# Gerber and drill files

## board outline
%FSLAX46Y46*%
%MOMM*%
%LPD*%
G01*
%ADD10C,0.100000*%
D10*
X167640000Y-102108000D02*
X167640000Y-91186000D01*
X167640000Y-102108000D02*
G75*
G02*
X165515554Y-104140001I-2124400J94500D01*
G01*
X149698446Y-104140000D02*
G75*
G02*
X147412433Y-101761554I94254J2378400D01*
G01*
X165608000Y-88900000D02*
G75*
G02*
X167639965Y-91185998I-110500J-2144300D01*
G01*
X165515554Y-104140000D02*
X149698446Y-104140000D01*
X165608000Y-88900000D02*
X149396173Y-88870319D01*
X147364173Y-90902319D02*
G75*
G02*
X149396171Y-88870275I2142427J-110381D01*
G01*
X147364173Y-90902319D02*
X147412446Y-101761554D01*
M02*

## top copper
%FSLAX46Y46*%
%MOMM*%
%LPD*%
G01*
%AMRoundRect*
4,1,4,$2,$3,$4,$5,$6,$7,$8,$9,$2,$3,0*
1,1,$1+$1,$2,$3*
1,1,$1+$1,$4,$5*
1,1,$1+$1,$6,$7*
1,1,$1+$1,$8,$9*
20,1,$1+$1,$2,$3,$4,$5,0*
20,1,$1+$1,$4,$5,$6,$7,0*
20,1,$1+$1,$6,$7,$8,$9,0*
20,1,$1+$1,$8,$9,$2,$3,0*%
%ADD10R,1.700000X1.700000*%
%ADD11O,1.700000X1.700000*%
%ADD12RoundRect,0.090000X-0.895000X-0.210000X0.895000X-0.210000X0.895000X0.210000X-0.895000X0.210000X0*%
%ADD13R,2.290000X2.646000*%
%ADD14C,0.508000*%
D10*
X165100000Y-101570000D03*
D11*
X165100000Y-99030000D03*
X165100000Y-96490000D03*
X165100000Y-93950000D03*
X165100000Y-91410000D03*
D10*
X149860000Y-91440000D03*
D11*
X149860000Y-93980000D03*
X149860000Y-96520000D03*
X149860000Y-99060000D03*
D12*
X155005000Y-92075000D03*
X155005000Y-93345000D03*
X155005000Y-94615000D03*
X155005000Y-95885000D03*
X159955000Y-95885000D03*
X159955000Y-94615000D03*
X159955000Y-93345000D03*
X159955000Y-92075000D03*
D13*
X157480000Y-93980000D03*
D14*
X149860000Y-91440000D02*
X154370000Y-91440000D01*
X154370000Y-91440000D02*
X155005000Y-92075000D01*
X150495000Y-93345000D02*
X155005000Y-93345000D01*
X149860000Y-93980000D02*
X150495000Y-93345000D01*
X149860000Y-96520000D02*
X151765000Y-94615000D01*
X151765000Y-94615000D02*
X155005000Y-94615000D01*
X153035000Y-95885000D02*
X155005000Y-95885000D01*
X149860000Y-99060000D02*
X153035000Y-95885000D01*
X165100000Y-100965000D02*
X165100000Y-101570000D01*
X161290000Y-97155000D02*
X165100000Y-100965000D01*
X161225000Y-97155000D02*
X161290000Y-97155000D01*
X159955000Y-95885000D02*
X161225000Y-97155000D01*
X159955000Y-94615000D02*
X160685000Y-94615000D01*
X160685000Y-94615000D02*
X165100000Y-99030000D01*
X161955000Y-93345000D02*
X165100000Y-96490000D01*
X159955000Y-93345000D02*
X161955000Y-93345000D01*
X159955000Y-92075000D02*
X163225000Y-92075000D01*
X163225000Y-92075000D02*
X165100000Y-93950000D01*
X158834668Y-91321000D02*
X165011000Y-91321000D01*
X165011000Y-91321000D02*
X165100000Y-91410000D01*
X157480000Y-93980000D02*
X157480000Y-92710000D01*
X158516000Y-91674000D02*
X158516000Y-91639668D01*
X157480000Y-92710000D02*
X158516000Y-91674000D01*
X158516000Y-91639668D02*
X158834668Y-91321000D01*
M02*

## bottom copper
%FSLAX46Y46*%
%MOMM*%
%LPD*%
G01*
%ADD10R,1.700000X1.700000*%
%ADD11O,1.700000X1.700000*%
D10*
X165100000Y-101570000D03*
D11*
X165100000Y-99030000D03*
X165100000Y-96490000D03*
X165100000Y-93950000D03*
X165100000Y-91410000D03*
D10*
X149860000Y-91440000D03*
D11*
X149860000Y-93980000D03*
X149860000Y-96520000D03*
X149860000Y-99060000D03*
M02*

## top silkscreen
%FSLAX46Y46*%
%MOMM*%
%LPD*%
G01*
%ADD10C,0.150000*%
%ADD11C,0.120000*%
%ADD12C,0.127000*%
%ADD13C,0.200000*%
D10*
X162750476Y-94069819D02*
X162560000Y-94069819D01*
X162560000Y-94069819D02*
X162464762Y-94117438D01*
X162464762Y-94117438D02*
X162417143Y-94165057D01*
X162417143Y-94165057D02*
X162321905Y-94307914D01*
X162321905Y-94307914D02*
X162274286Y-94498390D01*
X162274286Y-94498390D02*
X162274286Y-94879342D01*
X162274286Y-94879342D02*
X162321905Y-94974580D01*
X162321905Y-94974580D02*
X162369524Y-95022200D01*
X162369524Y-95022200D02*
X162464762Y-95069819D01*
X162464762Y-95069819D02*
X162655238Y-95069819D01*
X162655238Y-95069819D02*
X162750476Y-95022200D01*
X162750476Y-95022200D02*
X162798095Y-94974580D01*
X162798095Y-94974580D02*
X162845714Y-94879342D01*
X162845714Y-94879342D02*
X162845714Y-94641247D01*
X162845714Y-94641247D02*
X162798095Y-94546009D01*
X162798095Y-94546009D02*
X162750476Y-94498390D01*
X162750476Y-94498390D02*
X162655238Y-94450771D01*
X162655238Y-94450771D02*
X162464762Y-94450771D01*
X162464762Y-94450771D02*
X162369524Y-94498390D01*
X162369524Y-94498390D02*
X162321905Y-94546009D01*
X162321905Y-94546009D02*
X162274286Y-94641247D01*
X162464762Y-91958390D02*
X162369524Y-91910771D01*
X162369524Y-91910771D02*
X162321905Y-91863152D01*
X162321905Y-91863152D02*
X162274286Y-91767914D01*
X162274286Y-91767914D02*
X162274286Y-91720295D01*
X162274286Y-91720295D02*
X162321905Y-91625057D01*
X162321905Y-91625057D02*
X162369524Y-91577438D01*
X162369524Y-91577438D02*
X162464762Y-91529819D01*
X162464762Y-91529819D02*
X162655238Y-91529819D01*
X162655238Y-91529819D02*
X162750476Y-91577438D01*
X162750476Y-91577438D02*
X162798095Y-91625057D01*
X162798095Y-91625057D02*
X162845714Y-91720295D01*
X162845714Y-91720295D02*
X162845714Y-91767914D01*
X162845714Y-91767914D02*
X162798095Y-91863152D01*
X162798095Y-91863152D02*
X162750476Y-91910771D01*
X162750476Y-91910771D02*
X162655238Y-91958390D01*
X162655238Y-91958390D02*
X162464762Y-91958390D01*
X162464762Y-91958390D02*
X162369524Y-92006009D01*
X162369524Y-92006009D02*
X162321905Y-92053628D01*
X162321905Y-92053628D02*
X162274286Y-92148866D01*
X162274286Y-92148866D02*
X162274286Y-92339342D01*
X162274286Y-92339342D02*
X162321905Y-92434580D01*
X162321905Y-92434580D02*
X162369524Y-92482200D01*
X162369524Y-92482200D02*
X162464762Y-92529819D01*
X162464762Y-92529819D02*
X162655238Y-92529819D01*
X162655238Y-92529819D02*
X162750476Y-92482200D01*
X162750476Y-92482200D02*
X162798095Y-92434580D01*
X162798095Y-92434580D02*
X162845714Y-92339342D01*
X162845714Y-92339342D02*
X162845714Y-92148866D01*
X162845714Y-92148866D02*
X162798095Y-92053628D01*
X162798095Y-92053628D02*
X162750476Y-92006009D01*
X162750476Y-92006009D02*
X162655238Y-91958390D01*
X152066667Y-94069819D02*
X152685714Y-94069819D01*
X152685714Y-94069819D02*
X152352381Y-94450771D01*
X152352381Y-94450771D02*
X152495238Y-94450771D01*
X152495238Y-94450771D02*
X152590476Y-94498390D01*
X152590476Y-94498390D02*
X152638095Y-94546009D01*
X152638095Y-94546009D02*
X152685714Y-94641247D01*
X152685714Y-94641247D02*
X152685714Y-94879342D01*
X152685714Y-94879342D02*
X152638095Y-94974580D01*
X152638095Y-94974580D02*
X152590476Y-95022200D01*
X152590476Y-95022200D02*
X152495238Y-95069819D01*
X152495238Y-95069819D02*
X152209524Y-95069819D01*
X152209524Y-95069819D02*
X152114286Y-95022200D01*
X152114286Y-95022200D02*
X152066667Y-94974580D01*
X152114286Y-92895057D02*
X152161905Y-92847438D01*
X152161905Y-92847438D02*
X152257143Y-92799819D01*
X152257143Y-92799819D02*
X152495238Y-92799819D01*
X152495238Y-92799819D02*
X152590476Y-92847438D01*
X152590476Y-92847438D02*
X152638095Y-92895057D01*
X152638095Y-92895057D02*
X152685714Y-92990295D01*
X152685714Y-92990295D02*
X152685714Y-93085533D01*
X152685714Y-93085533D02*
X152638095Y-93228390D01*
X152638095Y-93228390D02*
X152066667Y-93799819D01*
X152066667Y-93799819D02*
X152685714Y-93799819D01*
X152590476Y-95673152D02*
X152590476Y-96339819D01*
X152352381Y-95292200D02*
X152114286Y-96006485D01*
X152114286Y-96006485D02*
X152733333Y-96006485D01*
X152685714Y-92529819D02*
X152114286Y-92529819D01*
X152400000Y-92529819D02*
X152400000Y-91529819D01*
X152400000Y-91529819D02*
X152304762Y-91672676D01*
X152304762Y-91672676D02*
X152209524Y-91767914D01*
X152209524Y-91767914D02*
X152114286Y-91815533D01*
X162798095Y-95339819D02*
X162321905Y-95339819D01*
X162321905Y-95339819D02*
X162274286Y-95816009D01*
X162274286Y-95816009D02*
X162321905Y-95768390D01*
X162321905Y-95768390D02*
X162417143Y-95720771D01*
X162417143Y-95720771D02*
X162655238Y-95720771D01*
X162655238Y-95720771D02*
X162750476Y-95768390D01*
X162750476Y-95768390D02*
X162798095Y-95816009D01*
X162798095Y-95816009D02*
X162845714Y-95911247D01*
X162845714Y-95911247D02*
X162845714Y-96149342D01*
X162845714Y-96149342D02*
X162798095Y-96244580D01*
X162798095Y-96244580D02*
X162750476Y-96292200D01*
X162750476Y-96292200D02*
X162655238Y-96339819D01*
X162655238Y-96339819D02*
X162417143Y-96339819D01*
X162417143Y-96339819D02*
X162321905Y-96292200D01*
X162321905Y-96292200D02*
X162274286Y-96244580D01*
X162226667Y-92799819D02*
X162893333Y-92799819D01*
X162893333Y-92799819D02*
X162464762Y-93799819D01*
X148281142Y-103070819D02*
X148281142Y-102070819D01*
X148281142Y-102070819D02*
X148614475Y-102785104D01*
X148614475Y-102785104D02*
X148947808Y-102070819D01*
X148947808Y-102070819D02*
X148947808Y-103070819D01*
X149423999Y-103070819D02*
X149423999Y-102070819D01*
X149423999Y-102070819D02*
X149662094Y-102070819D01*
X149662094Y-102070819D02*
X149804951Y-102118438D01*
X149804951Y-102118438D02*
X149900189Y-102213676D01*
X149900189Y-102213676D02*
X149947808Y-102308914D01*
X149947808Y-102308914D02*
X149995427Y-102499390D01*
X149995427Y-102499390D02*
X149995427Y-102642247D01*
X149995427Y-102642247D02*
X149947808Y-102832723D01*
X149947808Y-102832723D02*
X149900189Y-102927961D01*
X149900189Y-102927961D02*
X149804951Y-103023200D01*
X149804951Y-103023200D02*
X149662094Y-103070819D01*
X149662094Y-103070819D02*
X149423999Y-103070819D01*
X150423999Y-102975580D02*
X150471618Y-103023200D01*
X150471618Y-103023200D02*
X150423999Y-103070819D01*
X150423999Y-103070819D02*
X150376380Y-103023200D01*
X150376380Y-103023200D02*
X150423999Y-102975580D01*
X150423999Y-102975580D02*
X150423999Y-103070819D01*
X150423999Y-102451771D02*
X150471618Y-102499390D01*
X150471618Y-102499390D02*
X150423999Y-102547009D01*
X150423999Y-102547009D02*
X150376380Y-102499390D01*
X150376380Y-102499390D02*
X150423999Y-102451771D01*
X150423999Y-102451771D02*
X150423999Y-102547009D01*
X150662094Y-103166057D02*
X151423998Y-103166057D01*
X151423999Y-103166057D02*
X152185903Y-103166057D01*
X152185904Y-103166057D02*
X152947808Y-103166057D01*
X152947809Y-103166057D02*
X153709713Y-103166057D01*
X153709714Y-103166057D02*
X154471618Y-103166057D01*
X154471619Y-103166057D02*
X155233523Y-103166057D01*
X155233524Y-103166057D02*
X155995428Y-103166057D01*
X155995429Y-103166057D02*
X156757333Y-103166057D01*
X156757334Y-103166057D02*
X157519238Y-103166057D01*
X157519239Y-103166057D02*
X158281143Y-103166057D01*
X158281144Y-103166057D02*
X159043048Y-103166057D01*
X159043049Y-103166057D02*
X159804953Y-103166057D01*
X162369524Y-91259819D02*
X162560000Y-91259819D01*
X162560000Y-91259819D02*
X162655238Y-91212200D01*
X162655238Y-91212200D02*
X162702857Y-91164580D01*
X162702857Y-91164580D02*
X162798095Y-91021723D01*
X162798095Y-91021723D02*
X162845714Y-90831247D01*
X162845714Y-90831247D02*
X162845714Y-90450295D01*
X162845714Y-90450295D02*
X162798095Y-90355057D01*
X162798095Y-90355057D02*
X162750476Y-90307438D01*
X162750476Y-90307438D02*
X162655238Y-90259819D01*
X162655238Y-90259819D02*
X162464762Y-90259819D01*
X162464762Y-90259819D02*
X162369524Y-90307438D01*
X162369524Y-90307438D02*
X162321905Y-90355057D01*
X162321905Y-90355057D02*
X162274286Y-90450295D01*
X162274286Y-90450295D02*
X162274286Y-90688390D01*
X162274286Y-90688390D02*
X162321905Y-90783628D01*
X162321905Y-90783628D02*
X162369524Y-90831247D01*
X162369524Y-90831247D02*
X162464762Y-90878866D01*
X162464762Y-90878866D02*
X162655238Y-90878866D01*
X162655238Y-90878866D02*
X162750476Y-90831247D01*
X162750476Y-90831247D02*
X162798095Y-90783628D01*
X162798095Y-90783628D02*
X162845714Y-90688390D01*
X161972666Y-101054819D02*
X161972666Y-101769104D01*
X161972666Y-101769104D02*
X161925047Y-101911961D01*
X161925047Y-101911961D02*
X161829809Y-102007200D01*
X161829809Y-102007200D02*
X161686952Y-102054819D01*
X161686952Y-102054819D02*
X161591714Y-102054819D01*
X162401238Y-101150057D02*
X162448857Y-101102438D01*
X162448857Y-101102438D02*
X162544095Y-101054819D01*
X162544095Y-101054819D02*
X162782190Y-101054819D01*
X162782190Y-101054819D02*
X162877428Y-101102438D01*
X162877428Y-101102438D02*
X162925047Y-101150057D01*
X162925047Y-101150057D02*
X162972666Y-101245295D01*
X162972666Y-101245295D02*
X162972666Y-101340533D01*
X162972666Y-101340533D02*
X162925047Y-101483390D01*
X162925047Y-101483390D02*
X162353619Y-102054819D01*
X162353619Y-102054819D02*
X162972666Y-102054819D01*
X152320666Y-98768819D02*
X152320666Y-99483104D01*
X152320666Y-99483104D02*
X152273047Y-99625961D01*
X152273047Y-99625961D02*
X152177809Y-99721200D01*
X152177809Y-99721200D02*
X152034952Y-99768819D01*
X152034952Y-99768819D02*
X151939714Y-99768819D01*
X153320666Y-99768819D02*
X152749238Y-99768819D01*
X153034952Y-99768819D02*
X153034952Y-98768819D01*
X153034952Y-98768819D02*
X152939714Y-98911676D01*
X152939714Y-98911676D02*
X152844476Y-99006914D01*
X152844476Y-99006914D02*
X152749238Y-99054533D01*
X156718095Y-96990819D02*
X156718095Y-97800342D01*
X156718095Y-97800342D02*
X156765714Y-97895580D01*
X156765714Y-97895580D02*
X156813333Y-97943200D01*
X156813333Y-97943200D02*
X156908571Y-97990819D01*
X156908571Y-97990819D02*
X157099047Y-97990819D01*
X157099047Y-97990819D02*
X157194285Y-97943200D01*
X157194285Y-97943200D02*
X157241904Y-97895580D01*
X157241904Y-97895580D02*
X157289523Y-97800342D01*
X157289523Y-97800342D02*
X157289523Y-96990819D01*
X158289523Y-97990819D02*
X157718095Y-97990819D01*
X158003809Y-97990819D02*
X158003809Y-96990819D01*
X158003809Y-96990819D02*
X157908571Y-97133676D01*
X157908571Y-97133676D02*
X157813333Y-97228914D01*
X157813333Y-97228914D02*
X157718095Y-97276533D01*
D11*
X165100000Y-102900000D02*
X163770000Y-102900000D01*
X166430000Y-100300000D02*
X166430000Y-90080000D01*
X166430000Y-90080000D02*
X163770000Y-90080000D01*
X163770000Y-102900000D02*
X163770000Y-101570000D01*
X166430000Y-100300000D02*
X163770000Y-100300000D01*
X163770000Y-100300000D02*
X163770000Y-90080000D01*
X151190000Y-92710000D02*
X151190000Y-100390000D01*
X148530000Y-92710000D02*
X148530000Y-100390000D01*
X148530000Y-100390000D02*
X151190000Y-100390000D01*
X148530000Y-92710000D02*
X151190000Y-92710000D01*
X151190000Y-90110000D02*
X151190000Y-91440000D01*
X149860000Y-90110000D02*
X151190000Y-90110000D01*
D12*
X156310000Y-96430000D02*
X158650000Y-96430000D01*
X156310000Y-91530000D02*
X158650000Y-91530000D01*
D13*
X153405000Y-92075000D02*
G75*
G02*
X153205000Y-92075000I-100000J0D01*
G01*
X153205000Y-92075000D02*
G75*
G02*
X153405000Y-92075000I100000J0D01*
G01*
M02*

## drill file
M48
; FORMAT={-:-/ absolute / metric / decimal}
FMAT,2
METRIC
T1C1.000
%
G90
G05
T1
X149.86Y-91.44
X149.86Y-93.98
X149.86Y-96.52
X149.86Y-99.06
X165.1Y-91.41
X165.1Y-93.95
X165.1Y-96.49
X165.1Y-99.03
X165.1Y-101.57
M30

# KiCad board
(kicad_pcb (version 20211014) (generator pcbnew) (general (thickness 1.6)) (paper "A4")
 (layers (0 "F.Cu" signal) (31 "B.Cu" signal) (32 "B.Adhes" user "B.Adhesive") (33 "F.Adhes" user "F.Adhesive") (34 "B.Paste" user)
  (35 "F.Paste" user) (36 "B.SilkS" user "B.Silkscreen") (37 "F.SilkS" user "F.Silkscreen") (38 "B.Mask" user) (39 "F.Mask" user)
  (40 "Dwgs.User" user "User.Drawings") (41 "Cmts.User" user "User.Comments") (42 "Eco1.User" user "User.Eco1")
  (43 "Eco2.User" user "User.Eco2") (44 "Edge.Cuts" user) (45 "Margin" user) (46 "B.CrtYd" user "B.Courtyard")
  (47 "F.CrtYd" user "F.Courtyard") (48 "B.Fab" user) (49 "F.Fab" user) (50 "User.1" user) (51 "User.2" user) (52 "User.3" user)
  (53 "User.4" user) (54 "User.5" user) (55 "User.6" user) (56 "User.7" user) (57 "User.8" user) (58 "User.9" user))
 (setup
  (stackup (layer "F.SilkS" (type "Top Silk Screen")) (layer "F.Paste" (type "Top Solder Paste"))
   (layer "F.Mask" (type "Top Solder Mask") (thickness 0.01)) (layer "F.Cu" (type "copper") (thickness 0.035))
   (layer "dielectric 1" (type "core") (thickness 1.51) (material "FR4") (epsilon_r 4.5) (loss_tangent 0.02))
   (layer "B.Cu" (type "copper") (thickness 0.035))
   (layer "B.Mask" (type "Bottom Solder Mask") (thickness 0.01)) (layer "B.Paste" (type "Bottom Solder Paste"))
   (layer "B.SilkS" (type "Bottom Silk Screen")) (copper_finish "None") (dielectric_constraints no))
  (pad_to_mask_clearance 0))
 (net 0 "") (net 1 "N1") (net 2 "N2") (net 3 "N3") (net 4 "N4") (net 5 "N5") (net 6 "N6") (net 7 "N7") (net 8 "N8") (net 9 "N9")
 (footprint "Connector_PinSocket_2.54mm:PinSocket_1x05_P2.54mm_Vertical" (layer "F.Cu") (at 165.1 101.57 180)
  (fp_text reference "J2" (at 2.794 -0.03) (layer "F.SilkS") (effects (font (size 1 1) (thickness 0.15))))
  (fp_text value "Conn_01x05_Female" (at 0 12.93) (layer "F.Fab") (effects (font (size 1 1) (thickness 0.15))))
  (fp_line (start 0 -1.33) (end 1.33 -1.33) (layer "F.SilkS") (width 0.12))
  (fp_line (start -1.33 1.27) (end -1.33 11.49) (layer "F.SilkS") (width 0.12))
  (fp_line (start -1.33 11.49) (end 1.33 11.49) (layer "F.SilkS") (width 0.12))
  (fp_line (start 1.33 -1.33) (end 1.33 0) (layer "F.SilkS") (width 0.12))
  (fp_line (start -1.33 1.27) (end 1.33 1.27) (layer "F.SilkS") (width 0.12))
  (fp_line (start 1.33 1.27) (end 1.33 11.49) (layer "F.SilkS") (width 0.12))
  (pad "1" thru_hole rect (at 0 0 180) (size 1.7 1.7) (drill 1) (layers *.Cu *.Mask) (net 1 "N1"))
  (pad "2" thru_hole oval (at 0 2.54 180) (size 1.7 1.7) (drill 1) (layers *.Cu *.Mask) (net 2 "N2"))
  (pad "3" thru_hole oval (at 0 5.08 180) (size 1.7 1.7) (drill 1) (layers *.Cu *.Mask) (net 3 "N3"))
  (pad "4" thru_hole oval (at 0 7.62 180) (size 1.7 1.7) (drill 1) (layers *.Cu *.Mask) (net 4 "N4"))
  (pad "5" thru_hole oval (at 0 10.16 180) (size 1.7 1.7) (drill 1) (layers *.Cu *.Mask) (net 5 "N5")))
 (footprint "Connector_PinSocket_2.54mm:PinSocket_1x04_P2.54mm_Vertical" (layer "F.Cu") (at 149.86 91.44)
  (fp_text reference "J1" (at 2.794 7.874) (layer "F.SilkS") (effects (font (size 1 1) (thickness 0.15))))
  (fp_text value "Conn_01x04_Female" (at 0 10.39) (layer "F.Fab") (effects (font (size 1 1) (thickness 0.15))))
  (fp_line (start 1.33 1.27) (end 1.33 8.95) (layer "F.SilkS") (width 0.12))
  (fp_line (start -1.33 1.27) (end -1.33 8.95) (layer "F.SilkS") (width 0.12))
  (fp_line (start -1.33 8.95) (end 1.33 8.95) (layer "F.SilkS") (width 0.12))
  (fp_line (start -1.33 1.27) (end 1.33 1.27) (layer "F.SilkS") (width 0.12))
  (fp_line (start 1.33 -1.33) (end 1.33 0) (layer "F.SilkS") (width 0.12))
  (fp_line (start 0 -1.33) (end 1.33 -1.33) (layer "F.SilkS") (width 0.12))
  (pad "1" thru_hole rect (at 0 0) (size 1.7 1.7) (drill 1) (layers *.Cu *.Mask) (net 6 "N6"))
  (pad "2" thru_hole oval (at 0 2.54) (size 1.7 1.7) (drill 1) (layers *.Cu *.Mask) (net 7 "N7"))
  (pad "3" thru_hole oval (at 0 5.08) (size 1.7 1.7) (drill 1) (layers *.Cu *.Mask) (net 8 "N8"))
  (pad "4" thru_hole oval (at 0 7.62) (size 1.7 1.7) (drill 1) (layers *.Cu *.Mask) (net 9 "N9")))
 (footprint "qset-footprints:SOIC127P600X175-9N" (layer "F.Cu") (at 157.48 93.98)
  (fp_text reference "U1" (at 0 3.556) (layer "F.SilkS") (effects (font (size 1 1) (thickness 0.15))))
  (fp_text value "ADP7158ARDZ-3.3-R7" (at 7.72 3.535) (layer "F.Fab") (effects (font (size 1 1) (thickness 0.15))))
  (fp_line (start -1.17 2.45) (end 1.17 2.45) (layer "F.SilkS") (width 0.127))
  (fp_line (start -1.17 -2.45) (end 1.17 -2.45) (layer "F.SilkS") (width 0.127))
  (fp_circle (center -4.175 -1.905) (end -4.075 -1.905) (layer "F.SilkS") (width 0.2) (fill none))
  (pad "1" smd roundrect locked (at -2.475 -1.905) (size 1.97 0.6) (layers "F.Cu" "F.Paste" "F.Mask") (roundrect_rratio 0.15) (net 6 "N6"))
  (pad "2" smd roundrect locked (at -2.475 -0.635) (size 1.97 0.6) (layers "F.Cu" "F.Paste" "F.Mask") (roundrect_rratio 0.15) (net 7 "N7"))
  (pad "3" smd roundrect locked (at -2.475 0.635) (size 1.97 0.6) (layers "F.Cu" "F.Paste" "F.Mask") (roundrect_rratio 0.15) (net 8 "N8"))
  (pad "4" smd roundrect locked (at -2.475 1.905) (size 1.97 0.6) (layers "F.Cu" "F.Paste" "F.Mask") (roundrect_rratio 0.15) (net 9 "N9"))
  (pad "5" smd roundrect locked (at 2.475 1.905) (size 1.97 0.6) (layers "F.Cu" "F.Paste" "F.Mask") (roundrect_rratio 0.15) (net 1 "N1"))
  (pad "6" smd roundrect locked (at 2.475 0.635) (size 1.97 0.6) (layers "F.Cu" "F.Paste" "F.Mask") (roundrect_rratio 0.15) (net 2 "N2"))
  (pad "7" smd roundrect locked (at 2.475 -0.635) (size 1.97 0.6) (layers "F.Cu" "F.Paste" "F.Mask") (roundrect_rratio 0.15) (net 3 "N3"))
  (pad "8" smd roundrect locked (at 2.475 -1.905) (size 1.97 0.6) (layers "F.Cu" "F.Paste" "F.Mask") (roundrect_rratio 0.15) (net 4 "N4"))
  (pad "9" smd rect locked (at 0 0) (size 2.29 2.646) (layers "F.Cu" "F.Paste" "F.Mask") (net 5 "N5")))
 (gr_line (start 167.64 102.108) (end 167.64 91.186) (layer "Edge.Cuts") (width 0.1))
 (gr_arc (start 167.64 102.108) (mid 166.985443 103.550213) (end 165.515554 104.14) (layer "Edge.Cuts") (width 0.1))
 (gr_arc (start 149.698446 104.14) (mid 148.076596 103.411015) (end 147.412446 101.761554) (layer "Edge.Cuts") (width 0.1))
 (gr_arc (start 165.608 88.9) (mid 167.102319 89.617827) (end 167.64 91.186) (layer "Edge.Cuts") (width 0.1))
 (gr_line (start 165.515554 104.14) (end 149.698446 104.14) (layer "Edge.Cuts") (width 0.1))
 (gr_line (start 165.608 88.9) (end 149.396173 88.870319) (layer "Edge.Cuts") (width 0.1))
 (gr_arc (start 147.364173 90.902319) (mid 147.989659 89.495805) (end 149.396173 88.870319) (layer "Edge.Cuts") (width 0.1))
 (gr_line (start 147.364173 90.902319) (end 147.412446 101.761554) (layer "Edge.Cuts") (width 0.1))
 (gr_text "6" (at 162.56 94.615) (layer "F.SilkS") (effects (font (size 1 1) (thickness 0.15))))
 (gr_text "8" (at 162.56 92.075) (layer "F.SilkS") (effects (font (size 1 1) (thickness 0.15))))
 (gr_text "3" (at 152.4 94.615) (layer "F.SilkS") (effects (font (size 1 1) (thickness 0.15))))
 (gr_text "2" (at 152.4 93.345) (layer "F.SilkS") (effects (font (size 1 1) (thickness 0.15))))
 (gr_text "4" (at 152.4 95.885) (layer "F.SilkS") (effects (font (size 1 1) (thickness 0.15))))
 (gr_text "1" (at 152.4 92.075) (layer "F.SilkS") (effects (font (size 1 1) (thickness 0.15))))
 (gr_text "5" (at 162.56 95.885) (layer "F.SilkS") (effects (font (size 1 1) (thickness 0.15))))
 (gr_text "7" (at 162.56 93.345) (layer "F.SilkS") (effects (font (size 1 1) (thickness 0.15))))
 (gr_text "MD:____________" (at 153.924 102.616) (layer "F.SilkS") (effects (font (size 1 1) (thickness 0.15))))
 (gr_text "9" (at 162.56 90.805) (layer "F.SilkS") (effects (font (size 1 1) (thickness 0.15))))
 (segment (start 149.86 91.44) (end 154.37 91.44) (width 0.508) (layer "F.Cu") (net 6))
 (segment (start 154.37 91.44) (end 155.005 92.075) (width 0.508) (layer "F.Cu") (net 6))
 (segment (start 150.495 93.345) (end 155.005 93.345) (width 0.508) (layer "F.Cu") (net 7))
 (segment (start 149.86 93.98) (end 150.495 93.345) (width 0.508) (layer "F.Cu") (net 7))
 (segment (start 149.86 96.52) (end 151.765 94.615) (width 0.508) (layer "F.Cu") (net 8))
 (segment (start 151.765 94.615) (end 155.005 94.615) (width 0.508) (layer "F.Cu") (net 8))
 (segment (start 153.035 95.885) (end 155.005 95.885) (width 0.508) (layer "F.Cu") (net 9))
 (segment (start 149.86 99.06) (end 153.035 95.885) (width 0.508) (layer "F.Cu") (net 9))
 (segment (start 165.1 100.965) (end 165.1 101.57) (width 0.508) (layer "F.Cu") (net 1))
 (segment (start 161.29 97.155) (end 165.1 100.965) (width 0.508) (layer "F.Cu") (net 1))
 (segment (start 161.225 97.155) (end 161.29 97.155) (width 0.508) (layer "F.Cu") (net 1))
 (segment (start 159.955 95.885) (end 161.225 97.155) (width 0.508) (layer "F.Cu") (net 1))
 (segment (start 159.955 94.615) (end 160.685 94.615) (width 0.508) (layer "F.Cu") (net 2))
 (segment (start 160.685 94.615) (end 165.1 99.03) (width 0.508) (layer "F.Cu") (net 2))
 (segment (start 161.955 93.345) (end 165.1 96.49) (width 0.508) (layer "F.Cu") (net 3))
 (segment (start 159.955 93.345) (end 161.955 93.345) (width 0.508) (layer "F.Cu") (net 3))
 (segment (start 159.955 92.075) (end 163.225 92.075) (width 0.508) (layer "F.Cu") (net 4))
 (segment (start 163.225 92.075) (end 165.1 93.95) (width 0.508) (layer "F.Cu") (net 4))
 (segment (start 158.834668 91.321) (end 165.011 91.321) (width 0.508) (layer "F.Cu") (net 5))
 (segment (start 165.011 91.321) (end 165.1 91.41) (width 0.508) (layer "F.Cu") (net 5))
 (segment (start 157.48 93.98) (end 157.48 92.71) (width 0.508) (layer "F.Cu") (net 5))
 (segment (start 158.516 91.674) (end 158.516 91.639668) (width 0.508) (layer "F.Cu") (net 5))
 (segment (start 157.48 92.71) (end 158.516 91.674) (width 0.508) (layer "F.Cu") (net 5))
 (segment (start 158.516 91.639668) (end 158.834668 91.321) (width 0.508) (layer "F.Cu") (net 5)))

